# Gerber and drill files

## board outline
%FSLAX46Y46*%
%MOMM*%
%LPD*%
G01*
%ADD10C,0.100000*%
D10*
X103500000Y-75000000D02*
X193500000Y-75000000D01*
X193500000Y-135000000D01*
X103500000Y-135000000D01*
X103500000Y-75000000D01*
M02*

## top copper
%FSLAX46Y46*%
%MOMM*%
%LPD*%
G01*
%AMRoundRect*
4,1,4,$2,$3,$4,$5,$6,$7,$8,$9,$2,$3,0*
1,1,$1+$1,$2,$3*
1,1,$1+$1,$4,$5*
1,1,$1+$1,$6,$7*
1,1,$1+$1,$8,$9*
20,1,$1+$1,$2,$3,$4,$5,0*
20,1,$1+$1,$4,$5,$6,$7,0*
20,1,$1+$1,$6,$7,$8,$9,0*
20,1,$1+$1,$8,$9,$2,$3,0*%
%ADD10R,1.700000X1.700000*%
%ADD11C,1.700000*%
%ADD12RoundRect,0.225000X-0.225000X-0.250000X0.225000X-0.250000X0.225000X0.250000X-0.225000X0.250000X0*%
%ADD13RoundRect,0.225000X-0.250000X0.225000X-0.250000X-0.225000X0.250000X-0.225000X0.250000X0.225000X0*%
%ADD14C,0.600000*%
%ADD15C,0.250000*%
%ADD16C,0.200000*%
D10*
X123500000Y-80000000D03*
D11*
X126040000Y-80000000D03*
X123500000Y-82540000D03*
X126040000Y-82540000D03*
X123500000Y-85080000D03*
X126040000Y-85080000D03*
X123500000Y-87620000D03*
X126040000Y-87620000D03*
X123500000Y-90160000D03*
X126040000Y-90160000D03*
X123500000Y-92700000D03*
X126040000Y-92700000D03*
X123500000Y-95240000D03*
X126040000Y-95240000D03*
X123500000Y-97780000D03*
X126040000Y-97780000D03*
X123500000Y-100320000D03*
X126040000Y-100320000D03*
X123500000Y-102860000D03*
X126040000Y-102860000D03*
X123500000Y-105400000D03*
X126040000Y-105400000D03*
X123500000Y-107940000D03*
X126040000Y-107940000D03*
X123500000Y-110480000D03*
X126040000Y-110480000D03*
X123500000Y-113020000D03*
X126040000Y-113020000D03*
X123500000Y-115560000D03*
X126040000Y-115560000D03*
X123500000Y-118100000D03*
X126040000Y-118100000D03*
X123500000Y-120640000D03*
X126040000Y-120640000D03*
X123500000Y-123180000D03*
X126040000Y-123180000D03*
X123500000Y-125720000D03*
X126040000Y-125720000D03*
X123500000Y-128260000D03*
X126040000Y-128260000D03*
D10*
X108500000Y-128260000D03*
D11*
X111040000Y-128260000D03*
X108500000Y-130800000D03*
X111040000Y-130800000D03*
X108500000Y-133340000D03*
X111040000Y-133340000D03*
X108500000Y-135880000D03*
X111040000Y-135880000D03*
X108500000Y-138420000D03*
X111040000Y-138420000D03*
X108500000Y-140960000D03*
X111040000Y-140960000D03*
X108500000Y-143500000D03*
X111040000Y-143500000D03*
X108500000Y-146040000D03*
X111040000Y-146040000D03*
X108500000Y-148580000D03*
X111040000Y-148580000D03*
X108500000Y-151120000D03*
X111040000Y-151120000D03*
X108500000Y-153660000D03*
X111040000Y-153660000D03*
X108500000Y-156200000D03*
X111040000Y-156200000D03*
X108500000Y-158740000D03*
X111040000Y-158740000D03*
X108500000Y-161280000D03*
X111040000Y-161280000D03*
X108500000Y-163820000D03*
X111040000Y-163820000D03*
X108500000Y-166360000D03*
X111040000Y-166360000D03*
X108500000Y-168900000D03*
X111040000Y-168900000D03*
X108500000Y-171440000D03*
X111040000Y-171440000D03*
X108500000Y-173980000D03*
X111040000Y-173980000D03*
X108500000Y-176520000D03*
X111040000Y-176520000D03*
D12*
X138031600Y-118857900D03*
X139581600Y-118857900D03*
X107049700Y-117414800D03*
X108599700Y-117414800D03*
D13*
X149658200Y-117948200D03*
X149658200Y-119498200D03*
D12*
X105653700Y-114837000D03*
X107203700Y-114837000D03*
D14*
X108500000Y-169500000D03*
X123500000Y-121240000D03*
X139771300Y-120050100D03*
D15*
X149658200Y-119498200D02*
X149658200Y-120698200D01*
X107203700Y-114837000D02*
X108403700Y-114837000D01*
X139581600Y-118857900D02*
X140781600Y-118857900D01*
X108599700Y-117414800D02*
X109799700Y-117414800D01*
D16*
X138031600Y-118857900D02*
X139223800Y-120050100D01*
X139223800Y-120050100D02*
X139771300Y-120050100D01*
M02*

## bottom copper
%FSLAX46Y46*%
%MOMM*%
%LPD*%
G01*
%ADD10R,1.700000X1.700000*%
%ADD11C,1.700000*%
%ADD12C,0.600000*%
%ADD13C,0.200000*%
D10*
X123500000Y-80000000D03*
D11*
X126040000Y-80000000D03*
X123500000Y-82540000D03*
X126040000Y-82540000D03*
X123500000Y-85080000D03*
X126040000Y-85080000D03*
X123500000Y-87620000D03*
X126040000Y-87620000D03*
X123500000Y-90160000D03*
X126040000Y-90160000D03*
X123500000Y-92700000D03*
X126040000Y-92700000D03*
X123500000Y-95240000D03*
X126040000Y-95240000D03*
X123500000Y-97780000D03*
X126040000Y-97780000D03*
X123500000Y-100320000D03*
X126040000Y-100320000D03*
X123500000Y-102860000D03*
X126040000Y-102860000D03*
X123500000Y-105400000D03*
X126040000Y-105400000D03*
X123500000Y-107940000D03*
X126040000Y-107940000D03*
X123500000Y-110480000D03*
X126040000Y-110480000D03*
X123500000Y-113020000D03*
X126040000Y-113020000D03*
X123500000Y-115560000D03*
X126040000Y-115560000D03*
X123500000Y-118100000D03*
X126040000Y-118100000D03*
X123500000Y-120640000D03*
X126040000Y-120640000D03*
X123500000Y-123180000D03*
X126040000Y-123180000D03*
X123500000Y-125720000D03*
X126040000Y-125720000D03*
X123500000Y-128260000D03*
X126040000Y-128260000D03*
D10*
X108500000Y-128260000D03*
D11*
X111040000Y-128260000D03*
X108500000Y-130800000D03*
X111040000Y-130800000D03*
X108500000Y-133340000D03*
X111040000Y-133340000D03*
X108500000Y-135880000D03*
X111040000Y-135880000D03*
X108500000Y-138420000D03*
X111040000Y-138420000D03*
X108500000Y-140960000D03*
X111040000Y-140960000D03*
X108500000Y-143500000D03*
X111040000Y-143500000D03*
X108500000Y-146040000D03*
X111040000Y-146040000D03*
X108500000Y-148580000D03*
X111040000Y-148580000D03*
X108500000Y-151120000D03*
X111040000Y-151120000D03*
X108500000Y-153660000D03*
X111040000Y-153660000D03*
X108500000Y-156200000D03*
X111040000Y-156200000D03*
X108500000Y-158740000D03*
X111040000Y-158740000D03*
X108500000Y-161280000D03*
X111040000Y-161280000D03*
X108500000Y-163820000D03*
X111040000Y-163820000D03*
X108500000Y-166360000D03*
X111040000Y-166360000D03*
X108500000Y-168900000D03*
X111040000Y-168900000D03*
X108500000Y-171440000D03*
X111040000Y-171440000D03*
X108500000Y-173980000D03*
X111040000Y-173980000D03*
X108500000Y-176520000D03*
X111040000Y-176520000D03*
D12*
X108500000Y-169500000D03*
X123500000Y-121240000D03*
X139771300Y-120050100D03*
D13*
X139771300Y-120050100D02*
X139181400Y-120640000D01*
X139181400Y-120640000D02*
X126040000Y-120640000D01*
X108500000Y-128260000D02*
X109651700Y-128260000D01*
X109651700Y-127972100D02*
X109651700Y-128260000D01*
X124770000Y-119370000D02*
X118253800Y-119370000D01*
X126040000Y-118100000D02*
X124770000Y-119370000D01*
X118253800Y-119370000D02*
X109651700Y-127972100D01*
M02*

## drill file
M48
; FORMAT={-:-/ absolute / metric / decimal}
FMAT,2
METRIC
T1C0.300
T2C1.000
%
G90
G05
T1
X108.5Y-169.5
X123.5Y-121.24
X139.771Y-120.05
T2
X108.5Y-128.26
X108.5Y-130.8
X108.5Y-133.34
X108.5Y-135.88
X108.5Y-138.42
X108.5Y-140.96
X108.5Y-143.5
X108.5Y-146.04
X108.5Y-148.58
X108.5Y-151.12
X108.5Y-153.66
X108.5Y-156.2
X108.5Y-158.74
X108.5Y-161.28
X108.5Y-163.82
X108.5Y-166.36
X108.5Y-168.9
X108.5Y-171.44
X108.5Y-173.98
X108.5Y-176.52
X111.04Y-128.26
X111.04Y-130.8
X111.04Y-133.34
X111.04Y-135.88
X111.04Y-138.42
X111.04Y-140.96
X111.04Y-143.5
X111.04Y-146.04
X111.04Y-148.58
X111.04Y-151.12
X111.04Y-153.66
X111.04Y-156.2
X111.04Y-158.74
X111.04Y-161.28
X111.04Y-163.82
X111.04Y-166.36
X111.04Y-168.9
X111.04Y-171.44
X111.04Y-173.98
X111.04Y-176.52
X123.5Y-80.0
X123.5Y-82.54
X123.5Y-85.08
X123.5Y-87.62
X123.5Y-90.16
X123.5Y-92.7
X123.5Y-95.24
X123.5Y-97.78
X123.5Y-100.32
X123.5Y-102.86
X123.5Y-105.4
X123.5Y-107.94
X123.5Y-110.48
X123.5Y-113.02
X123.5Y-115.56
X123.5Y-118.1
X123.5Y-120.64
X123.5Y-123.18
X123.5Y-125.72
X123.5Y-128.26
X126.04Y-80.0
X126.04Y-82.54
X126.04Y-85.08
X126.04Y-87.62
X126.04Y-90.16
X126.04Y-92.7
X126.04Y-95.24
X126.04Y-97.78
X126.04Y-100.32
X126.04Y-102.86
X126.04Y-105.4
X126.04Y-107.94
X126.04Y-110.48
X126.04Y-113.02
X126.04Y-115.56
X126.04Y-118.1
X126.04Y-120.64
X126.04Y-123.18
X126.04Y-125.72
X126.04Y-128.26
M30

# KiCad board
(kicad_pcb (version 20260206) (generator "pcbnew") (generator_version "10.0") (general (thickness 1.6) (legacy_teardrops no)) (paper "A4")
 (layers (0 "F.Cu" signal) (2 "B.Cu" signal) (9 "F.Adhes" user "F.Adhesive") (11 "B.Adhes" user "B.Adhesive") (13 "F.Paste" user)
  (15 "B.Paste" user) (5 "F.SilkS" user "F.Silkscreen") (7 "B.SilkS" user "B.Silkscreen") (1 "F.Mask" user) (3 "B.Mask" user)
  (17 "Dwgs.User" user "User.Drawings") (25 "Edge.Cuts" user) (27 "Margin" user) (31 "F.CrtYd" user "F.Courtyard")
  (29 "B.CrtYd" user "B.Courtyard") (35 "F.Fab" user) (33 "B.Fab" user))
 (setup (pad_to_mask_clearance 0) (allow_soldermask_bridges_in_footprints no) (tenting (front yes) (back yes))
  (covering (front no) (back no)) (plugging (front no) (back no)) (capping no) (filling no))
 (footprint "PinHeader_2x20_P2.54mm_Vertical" (layer "F.Cu") (at 123.5 80)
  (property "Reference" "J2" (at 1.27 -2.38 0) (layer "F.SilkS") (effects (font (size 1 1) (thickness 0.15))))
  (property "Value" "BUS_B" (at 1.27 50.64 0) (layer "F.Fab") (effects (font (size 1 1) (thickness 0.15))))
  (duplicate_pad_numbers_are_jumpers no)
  (pad "1" thru_hole rect (at 0 0) (size 1.7 1.7) (drill 1) (layers "*.Cu" "*.Mask") (remove_unused_layers no) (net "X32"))
  (pad "2" thru_hole circle (at 2.54 0) (size 1.7 1.7) (drill 1) (layers "*.Cu" "*.Mask") (remove_unused_layers no) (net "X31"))
  (pad "3" thru_hole circle (at 0 2.54) (size 1.7 1.7) (drill 1) (layers "*.Cu" "*.Mask") (remove_unused_layers no) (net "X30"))
  (pad "4" thru_hole circle (at 2.54 2.54) (size 1.7 1.7) (drill 1) (layers "*.Cu" "*.Mask") (remove_unused_layers no) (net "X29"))
  (pad "5" thru_hole circle (at 0 5.08) (size 1.7 1.7) (drill 1) (layers "*.Cu" "*.Mask") (remove_unused_layers no) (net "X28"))
  (pad "6" thru_hole circle (at 2.54 5.08) (size 1.7 1.7) (drill 1) (layers "*.Cu" "*.Mask") (remove_unused_layers no) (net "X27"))
  (pad "7" thru_hole circle (at 0 7.62) (size 1.7 1.7) (drill 1) (layers "*.Cu" "*.Mask") (remove_unused_layers no) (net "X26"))
  (pad "8" thru_hole circle (at 2.54 7.62) (size 1.7 1.7) (drill 1) (layers "*.Cu" "*.Mask") (remove_unused_layers no) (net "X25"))
  (pad "9" thru_hole circle (at 0 10.16) (size 1.7 1.7) (drill 1) (layers "*.Cu" "*.Mask") (remove_unused_layers no) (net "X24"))
  (pad "10" thru_hole circle (at 2.54 10.16) (size 1.7 1.7) (drill 1) (layers "*.Cu" "*.Mask") (remove_unused_layers no) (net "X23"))
  (pad "11" thru_hole circle (at 0 12.7) (size 1.7 1.7) (drill 1) (layers "*.Cu" "*.Mask") (remove_unused_layers no) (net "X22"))
  (pad "12" thru_hole circle (at 2.54 12.7) (size 1.7 1.7) (drill 1) (layers "*.Cu" "*.Mask") (remove_unused_layers no) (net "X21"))
  (pad "13" thru_hole circle (at 0 15.24) (size 1.7 1.7) (drill 1) (layers "*.Cu" "*.Mask") (remove_unused_layers no) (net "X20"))
  (pad "14" thru_hole circle (at 2.54 15.24) (size 1.7 1.7) (drill 1) (layers "*.Cu" "*.Mask") (remove_unused_layers no) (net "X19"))
  (pad "15" thru_hole circle (at 0 17.78) (size 1.7 1.7) (drill 1) (layers "*.Cu" "*.Mask") (remove_unused_layers no) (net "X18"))
  (pad "16" thru_hole circle (at 2.54 17.78) (size 1.7 1.7) (drill 1) (layers "*.Cu" "*.Mask") (remove_unused_layers no) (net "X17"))
  (pad "17" thru_hole circle (at 0 20.32) (size 1.7 1.7) (drill 1) (layers "*.Cu" "*.Mask") (remove_unused_layers no) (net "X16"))
  (pad "18" thru_hole circle (at 2.54 20.32) (size 1.7 1.7) (drill 1) (layers "*.Cu" "*.Mask") (remove_unused_layers no) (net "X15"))
  (pad "19" thru_hole circle (at 0 22.86) (size 1.7 1.7) (drill 1) (layers "*.Cu" "*.Mask") (remove_unused_layers no) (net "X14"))
  (pad "20" thru_hole circle (at 2.54 22.86) (size 1.7 1.7) (drill 1) (layers "*.Cu" "*.Mask") (remove_unused_layers no) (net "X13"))
  (pad "21" thru_hole circle (at 0 25.4) (size 1.7 1.7) (drill 1) (layers "*.Cu" "*.Mask") (remove_unused_layers no) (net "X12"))
  (pad "22" thru_hole circle (at 2.54 25.4) (size 1.7 1.7) (drill 1) (layers "*.Cu" "*.Mask") (remove_unused_layers no) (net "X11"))
  (pad "23" thru_hole circle (at 0 27.94) (size 1.7 1.7) (drill 1) (layers "*.Cu" "*.Mask") (remove_unused_layers no) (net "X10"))
  (pad "24" thru_hole circle (at 2.54 27.94) (size 1.7 1.7) (drill 1) (layers "*.Cu" "*.Mask") (remove_unused_layers no) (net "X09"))
  (pad "25" thru_hole circle (at 0 30.48) (size 1.7 1.7) (drill 1) (layers "*.Cu" "*.Mask") (remove_unused_layers no) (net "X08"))
  (pad "26" thru_hole circle (at 2.54 30.48) (size 1.7 1.7) (drill 1) (layers "*.Cu" "*.Mask") (remove_unused_layers no) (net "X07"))
  (pad "27" thru_hole circle (at 0 33.02) (size 1.7 1.7) (drill 1) (layers "*.Cu" "*.Mask") (remove_unused_layers no) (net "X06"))
  (pad "28" thru_hole circle (at 2.54 33.02) (size 1.7 1.7) (drill 1) (layers "*.Cu" "*.Mask") (remove_unused_layers no) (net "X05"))
  (pad "29" thru_hole circle (at 0 35.56) (size 1.7 1.7) (drill 1) (layers "*.Cu" "*.Mask") (remove_unused_layers no) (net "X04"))
  (pad "30" thru_hole circle (at 2.54 35.56) (size 1.7 1.7) (drill 1) (layers "*.Cu" "*.Mask") (remove_unused_layers no) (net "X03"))
  (pad "31" thru_hole circle (at 0 38.1) (size 1.7 1.7) (drill 1) (layers "*.Cu" "*.Mask") (remove_unused_layers no) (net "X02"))
  (pad "32" thru_hole circle (at 2.54 38.1) (size 1.7 1.7) (drill 1) (layers "*.Cu" "*.Mask") (remove_unused_layers no) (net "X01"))
  (pad "33" thru_hole circle (at 0 40.64) (size 1.7 1.7) (drill 1) (layers "*.Cu" "*.Mask") (remove_unused_layers no) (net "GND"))
  (pad "34" thru_hole circle (at 2.54 40.64) (size 1.7 1.7) (drill 1) (layers "*.Cu" "*.Mask") (remove_unused_layers no) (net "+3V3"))
  (pad "35" thru_hole circle (at 0 43.18) (size 1.7 1.7) (drill 1) (layers "*.Cu" "*.Mask") (remove_unused_layers no) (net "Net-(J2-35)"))
  (pad "36" thru_hole circle (at 2.54 43.18) (size 1.7 1.7) (drill 1) (layers "*.Cu" "*.Mask") (remove_unused_layers no) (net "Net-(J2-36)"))
  (pad "37" thru_hole circle (at 0 45.72) (size 1.7 1.7) (drill 1) (layers "*.Cu" "*.Mask") (remove_unused_layers no) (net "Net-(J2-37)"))
  (pad "38" thru_hole circle (at 2.54 45.72) (size 1.7 1.7) (drill 1) (layers "*.Cu" "*.Mask") (remove_unused_layers no) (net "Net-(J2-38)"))
  (pad "39" thru_hole circle (at 0 48.26) (size 1.7 1.7) (drill 1) (layers "*.Cu" "*.Mask") (remove_unused_layers no) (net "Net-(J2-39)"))
  (pad "40" thru_hole circle (at 2.54 48.26) (size 1.7 1.7) (drill 1) (layers "*.Cu" "*.Mask") (remove_unused_layers no) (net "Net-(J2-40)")))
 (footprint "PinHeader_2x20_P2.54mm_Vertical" (layer "F.Cu") (at 108.5 128.26)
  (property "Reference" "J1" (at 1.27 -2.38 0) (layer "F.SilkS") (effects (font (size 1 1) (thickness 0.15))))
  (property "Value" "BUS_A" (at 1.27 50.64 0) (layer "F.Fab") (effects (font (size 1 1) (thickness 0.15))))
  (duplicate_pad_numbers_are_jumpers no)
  (pad "1" thru_hole rect (at 0 0) (size 1.7 1.7) (drill 1) (layers "*.Cu" "*.Mask") (remove_unused_layers no) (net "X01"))
  (pad "2" thru_hole circle (at 2.54 0) (size 1.7 1.7) (drill 1) (layers "*.Cu" "*.Mask") (remove_unused_layers no) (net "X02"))
  (pad "3" thru_hole circle (at 0 2.54) (size 1.7 1.7) (drill 1) (layers "*.Cu" "*.Mask") (remove_unused_layers no) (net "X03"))
  (pad "4" thru_hole circle (at 2.54 2.54) (size 1.7 1.7) (drill 1) (layers "*.Cu" "*.Mask") (remove_unused_layers no) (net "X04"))
  (pad "5" thru_hole circle (at 0 5.08) (size 1.7 1.7) (drill 1) (layers "*.Cu" "*.Mask") (remove_unused_layers no) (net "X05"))
  (pad "6" thru_hole circle (at 2.54 5.08) (size 1.7 1.7) (drill 1) (layers "*.Cu" "*.Mask") (remove_unused_layers no) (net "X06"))
  (pad "7" thru_hole circle (at 0 7.62) (size 1.7 1.7) (drill 1) (layers "*.Cu" "*.Mask") (remove_unused_layers no) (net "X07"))
  (pad "8" thru_hole circle (at 2.54 7.62) (size 1.7 1.7) (drill 1) (layers "*.Cu" "*.Mask") (remove_unused_layers no) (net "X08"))
  (pad "9" thru_hole circle (at 0 10.16) (size 1.7 1.7) (drill 1) (layers "*.Cu" "*.Mask") (remove_unused_layers no) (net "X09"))
  (pad "10" thru_hole circle (at 2.54 10.16) (size 1.7 1.7) (drill 1) (layers "*.Cu" "*.Mask") (remove_unused_layers no) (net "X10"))
  (pad "11" thru_hole circle (at 0 12.7) (size 1.7 1.7) (drill 1) (layers "*.Cu" "*.Mask") (remove_unused_layers no) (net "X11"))
  (pad "12" thru_hole circle (at 2.54 12.7) (size 1.7 1.7) (drill 1) (layers "*.Cu" "*.Mask") (remove_unused_layers no) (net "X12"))
  (pad "13" thru_hole circle (at 0 15.24) (size 1.7 1.7) (drill 1) (layers "*.Cu" "*.Mask") (remove_unused_layers no) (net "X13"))
  (pad "14" thru_hole circle (at 2.54 15.24) (size 1.7 1.7) (drill 1) (layers "*.Cu" "*.Mask") (remove_unused_layers no) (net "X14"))
  (pad "15" thru_hole circle (at 0 17.78) (size 1.7 1.7) (drill 1) (layers "*.Cu" "*.Mask") (remove_unused_layers no) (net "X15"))
  (pad "16" thru_hole circle (at 2.54 17.78) (size 1.7 1.7) (drill 1) (layers "*.Cu" "*.Mask") (remove_unused_layers no) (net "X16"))
  (pad "17" thru_hole circle (at 0 20.32) (size 1.7 1.7) (drill 1) (layers "*.Cu" "*.Mask") (remove_unused_layers no) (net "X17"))
  (pad "18" thru_hole circle (at 2.54 20.32) (size 1.7 1.7) (drill 1) (layers "*.Cu" "*.Mask") (remove_unused_layers no) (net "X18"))
  (pad "19" thru_hole circle (at 0 22.86) (size 1.7 1.7) (drill 1) (layers "*.Cu" "*.Mask") (remove_unused_layers no) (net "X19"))
  (pad "20" thru_hole circle (at 2.54 22.86) (size 1.7 1.7) (drill 1) (layers "*.Cu" "*.Mask") (remove_unused_layers no) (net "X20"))
  (pad "21" thru_hole circle (at 0 25.4) (size 1.7 1.7) (drill 1) (layers "*.Cu" "*.Mask") (remove_unused_layers no) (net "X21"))
  (pad "22" thru_hole circle (at 2.54 25.4) (size 1.7 1.7) (drill 1) (layers "*.Cu" "*.Mask") (remove_unused_layers no) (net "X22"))
  (pad "23" thru_hole circle (at 0 27.94) (size 1.7 1.7) (drill 1) (layers "*.Cu" "*.Mask") (remove_unused_layers no) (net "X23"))
  (pad "24" thru_hole circle (at 2.54 27.94) (size 1.7 1.7) (drill 1) (layers "*.Cu" "*.Mask") (remove_unused_layers no) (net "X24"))
  (pad "25" thru_hole circle (at 0 30.48) (size 1.7 1.7) (drill 1) (layers "*.Cu" "*.Mask") (remove_unused_layers no) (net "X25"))
  (pad "26" thru_hole circle (at 2.54 30.48) (size 1.7 1.7) (drill 1) (layers "*.Cu" "*.Mask") (remove_unused_layers no) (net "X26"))
  (pad "27" thru_hole circle (at 0 33.02) (size 1.7 1.7) (drill 1) (layers "*.Cu" "*.Mask") (remove_unused_layers no) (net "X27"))
  (pad "28" thru_hole circle (at 2.54 33.02) (size 1.7 1.7) (drill 1) (layers "*.Cu" "*.Mask") (remove_unused_layers no) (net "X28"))
  (pad "29" thru_hole circle (at 0 35.56) (size 1.7 1.7) (drill 1) (layers "*.Cu" "*.Mask") (remove_unused_layers no) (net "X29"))
  (pad "30" thru_hole circle (at 2.54 35.56) (size 1.7 1.7) (drill 1) (layers "*.Cu" "*.Mask") (remove_unused_layers no) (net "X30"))
  (pad "31" thru_hole circle (at 0 38.1) (size 1.7 1.7) (drill 1) (layers "*.Cu" "*.Mask") (remove_unused_layers no) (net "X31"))
  (pad "32" thru_hole circle (at 2.54 38.1) (size 1.7 1.7) (drill 1) (layers "*.Cu" "*.Mask") (remove_unused_layers no) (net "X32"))
  (pad "33" thru_hole circle (at 0 40.64) (size 1.7 1.7) (drill 1) (layers "*.Cu" "*.Mask") (remove_unused_layers no) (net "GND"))
  (pad "34" thru_hole circle (at 2.54 40.64) (size 1.7 1.7) (drill 1) (layers "*.Cu" "*.Mask") (remove_unused_layers no) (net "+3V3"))
  (pad "35" thru_hole circle (at 0 43.18) (size 1.7 1.7) (drill 1) (layers "*.Cu" "*.Mask") (remove_unused_layers no) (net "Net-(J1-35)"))
  (pad "36" thru_hole circle (at 2.54 43.18) (size 1.7 1.7) (drill 1) (layers "*.Cu" "*.Mask") (remove_unused_layers no) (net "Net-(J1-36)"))
  (pad "37" thru_hole circle (at 0 45.72) (size 1.7 1.7) (drill 1) (layers "*.Cu" "*.Mask") (remove_unused_layers no) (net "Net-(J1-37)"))
  (pad "38" thru_hole circle (at 2.54 45.72) (size 1.7 1.7) (drill 1) (layers "*.Cu" "*.Mask") (remove_unused_layers no) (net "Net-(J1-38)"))
  (pad "39" thru_hole circle (at 0 48.26) (size 1.7 1.7) (drill 1) (layers "*.Cu" "*.Mask") (remove_unused_layers no) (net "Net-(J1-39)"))
  (pad "40" thru_hole circle (at 2.54 48.26) (size 1.7 1.7) (drill 1) (layers "*.Cu" "*.Mask") (remove_unused_layers no) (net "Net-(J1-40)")))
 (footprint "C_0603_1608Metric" (layer "F.Cu") (at 138.8066 118.8579)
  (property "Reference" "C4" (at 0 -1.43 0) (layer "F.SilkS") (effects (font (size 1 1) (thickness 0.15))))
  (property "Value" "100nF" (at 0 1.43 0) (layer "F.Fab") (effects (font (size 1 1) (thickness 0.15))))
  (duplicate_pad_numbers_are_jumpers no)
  (pad "1" smd roundrect (at -0.775 0) (size 0.9 0.95) (layers "F.Cu" "F.Mask" "F.Paste") (roundrect_rratio 0.25) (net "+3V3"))
  (pad "2" smd roundrect (at 0.775 0) (size 0.9 0.95) (layers "F.Cu" "F.Mask" "F.Paste") (roundrect_rratio 0.25) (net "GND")))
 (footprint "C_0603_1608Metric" (layer "F.Cu") (at 107.8247 117.4148)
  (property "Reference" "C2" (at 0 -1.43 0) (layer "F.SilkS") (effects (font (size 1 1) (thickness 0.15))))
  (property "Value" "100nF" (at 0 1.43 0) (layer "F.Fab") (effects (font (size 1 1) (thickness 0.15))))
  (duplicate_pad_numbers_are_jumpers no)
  (pad "1" smd roundrect (at -0.775 0) (size 0.9 0.95) (layers "F.Cu" "F.Mask" "F.Paste") (roundrect_rratio 0.25) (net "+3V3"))
  (pad "2" smd roundrect (at 0.775 0) (size 0.9 0.95) (layers "F.Cu" "F.Mask" "F.Paste") (roundrect_rratio 0.25) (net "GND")))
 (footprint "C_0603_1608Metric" (layer "F.Cu") (at 149.6582 118.7232 -90)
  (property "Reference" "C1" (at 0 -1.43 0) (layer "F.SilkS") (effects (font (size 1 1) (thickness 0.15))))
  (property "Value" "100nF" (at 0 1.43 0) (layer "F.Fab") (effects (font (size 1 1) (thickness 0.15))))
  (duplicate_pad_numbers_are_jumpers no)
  (pad "1" smd roundrect (at -0.775 0 270) (size 0.9 0.95) (layers "F.Cu" "F.Mask" "F.Paste") (roundrect_rratio 0.25) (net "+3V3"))
  (pad "2" smd roundrect (at 0.775 0 270) (size 0.9 0.95) (layers "F.Cu" "F.Mask" "F.Paste") (roundrect_rratio 0.25) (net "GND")))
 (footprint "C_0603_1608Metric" (layer "F.Cu") (at 106.4287 114.837)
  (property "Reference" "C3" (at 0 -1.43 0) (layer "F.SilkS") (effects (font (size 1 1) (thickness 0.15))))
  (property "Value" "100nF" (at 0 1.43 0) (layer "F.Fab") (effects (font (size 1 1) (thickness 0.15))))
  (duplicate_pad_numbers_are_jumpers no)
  (pad "1" smd roundrect (at -0.775 0) (size 0.9 0.95) (layers "F.Cu" "F.Mask" "F.Paste") (roundrect_rratio 0.25) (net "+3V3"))
  (pad "2" smd roundrect (at 0.775 0) (size 0.9 0.95) (layers "F.Cu" "F.Mask" "F.Paste") (roundrect_rratio 0.25) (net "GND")))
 (gr_rect (start 103.5 75) (end 193.5 135) (stroke (width 0.1) (type default)) (fill no) (layer "Edge.Cuts"))
 (segment (start 149.6582 119.4982) (end 149.6582 120.6982) (width 0.25) (layer "F.Cu") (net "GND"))
 (segment (start 107.2037 114.837) (end 108.4037 114.837) (width 0.25) (layer "F.Cu") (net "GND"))
 (segment (start 139.5816 118.8579) (end 140.7816 118.8579) (width 0.25) (layer "F.Cu") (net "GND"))
 (segment (start 108.5997 117.4148) (end 109.7997 117.4148) (width 0.25) (layer "F.Cu") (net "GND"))
 (via (at 108.5 169.5) (size 0.6) (drill 0.3) (layers "F.Cu" "B.Cu") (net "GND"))
 (via (at 123.5 121.24) (size 0.6) (drill 0.3) (layers "F.Cu" "B.Cu") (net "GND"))
 (segment (start 138.0316 118.8579) (end 139.2238 120.0501) (width 0.2) (layer "F.Cu") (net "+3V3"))
 (segment (start 139.2238 120.0501) (end 139.7713 120.0501) (width 0.2) (layer "F.Cu") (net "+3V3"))
 (via (at 139.7713 120.0501) (size 0.6) (drill 0.3) (layers "F.Cu" "B.Cu") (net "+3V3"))
 (segment (start 139.7713 120.0501) (end 139.1814 120.64) (width 0.2) (layer "B.Cu") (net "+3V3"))
 (segment (start 139.1814 120.64) (end 126.04 120.64) (width 0.2) (layer "B.Cu") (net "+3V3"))
 (segment (start 108.5 128.26) (end 109.6517 128.26) (width 0.2) (layer "B.Cu") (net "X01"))
 (segment (start 109.6517 127.9721) (end 109.6517 128.26) (width 0.2) (layer "B.Cu") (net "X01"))
 (segment (start 124.77 119.37) (end 118.2538 119.37) (width 0.2) (layer "B.Cu") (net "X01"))
 (segment (start 126.04 118.1) (end 124.77 119.37) (width 0.2) (layer "B.Cu") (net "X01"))
 (segment (start 118.2538 119.37) (end 109.6517 127.9721) (width 0.2) (layer "B.Cu") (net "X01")))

